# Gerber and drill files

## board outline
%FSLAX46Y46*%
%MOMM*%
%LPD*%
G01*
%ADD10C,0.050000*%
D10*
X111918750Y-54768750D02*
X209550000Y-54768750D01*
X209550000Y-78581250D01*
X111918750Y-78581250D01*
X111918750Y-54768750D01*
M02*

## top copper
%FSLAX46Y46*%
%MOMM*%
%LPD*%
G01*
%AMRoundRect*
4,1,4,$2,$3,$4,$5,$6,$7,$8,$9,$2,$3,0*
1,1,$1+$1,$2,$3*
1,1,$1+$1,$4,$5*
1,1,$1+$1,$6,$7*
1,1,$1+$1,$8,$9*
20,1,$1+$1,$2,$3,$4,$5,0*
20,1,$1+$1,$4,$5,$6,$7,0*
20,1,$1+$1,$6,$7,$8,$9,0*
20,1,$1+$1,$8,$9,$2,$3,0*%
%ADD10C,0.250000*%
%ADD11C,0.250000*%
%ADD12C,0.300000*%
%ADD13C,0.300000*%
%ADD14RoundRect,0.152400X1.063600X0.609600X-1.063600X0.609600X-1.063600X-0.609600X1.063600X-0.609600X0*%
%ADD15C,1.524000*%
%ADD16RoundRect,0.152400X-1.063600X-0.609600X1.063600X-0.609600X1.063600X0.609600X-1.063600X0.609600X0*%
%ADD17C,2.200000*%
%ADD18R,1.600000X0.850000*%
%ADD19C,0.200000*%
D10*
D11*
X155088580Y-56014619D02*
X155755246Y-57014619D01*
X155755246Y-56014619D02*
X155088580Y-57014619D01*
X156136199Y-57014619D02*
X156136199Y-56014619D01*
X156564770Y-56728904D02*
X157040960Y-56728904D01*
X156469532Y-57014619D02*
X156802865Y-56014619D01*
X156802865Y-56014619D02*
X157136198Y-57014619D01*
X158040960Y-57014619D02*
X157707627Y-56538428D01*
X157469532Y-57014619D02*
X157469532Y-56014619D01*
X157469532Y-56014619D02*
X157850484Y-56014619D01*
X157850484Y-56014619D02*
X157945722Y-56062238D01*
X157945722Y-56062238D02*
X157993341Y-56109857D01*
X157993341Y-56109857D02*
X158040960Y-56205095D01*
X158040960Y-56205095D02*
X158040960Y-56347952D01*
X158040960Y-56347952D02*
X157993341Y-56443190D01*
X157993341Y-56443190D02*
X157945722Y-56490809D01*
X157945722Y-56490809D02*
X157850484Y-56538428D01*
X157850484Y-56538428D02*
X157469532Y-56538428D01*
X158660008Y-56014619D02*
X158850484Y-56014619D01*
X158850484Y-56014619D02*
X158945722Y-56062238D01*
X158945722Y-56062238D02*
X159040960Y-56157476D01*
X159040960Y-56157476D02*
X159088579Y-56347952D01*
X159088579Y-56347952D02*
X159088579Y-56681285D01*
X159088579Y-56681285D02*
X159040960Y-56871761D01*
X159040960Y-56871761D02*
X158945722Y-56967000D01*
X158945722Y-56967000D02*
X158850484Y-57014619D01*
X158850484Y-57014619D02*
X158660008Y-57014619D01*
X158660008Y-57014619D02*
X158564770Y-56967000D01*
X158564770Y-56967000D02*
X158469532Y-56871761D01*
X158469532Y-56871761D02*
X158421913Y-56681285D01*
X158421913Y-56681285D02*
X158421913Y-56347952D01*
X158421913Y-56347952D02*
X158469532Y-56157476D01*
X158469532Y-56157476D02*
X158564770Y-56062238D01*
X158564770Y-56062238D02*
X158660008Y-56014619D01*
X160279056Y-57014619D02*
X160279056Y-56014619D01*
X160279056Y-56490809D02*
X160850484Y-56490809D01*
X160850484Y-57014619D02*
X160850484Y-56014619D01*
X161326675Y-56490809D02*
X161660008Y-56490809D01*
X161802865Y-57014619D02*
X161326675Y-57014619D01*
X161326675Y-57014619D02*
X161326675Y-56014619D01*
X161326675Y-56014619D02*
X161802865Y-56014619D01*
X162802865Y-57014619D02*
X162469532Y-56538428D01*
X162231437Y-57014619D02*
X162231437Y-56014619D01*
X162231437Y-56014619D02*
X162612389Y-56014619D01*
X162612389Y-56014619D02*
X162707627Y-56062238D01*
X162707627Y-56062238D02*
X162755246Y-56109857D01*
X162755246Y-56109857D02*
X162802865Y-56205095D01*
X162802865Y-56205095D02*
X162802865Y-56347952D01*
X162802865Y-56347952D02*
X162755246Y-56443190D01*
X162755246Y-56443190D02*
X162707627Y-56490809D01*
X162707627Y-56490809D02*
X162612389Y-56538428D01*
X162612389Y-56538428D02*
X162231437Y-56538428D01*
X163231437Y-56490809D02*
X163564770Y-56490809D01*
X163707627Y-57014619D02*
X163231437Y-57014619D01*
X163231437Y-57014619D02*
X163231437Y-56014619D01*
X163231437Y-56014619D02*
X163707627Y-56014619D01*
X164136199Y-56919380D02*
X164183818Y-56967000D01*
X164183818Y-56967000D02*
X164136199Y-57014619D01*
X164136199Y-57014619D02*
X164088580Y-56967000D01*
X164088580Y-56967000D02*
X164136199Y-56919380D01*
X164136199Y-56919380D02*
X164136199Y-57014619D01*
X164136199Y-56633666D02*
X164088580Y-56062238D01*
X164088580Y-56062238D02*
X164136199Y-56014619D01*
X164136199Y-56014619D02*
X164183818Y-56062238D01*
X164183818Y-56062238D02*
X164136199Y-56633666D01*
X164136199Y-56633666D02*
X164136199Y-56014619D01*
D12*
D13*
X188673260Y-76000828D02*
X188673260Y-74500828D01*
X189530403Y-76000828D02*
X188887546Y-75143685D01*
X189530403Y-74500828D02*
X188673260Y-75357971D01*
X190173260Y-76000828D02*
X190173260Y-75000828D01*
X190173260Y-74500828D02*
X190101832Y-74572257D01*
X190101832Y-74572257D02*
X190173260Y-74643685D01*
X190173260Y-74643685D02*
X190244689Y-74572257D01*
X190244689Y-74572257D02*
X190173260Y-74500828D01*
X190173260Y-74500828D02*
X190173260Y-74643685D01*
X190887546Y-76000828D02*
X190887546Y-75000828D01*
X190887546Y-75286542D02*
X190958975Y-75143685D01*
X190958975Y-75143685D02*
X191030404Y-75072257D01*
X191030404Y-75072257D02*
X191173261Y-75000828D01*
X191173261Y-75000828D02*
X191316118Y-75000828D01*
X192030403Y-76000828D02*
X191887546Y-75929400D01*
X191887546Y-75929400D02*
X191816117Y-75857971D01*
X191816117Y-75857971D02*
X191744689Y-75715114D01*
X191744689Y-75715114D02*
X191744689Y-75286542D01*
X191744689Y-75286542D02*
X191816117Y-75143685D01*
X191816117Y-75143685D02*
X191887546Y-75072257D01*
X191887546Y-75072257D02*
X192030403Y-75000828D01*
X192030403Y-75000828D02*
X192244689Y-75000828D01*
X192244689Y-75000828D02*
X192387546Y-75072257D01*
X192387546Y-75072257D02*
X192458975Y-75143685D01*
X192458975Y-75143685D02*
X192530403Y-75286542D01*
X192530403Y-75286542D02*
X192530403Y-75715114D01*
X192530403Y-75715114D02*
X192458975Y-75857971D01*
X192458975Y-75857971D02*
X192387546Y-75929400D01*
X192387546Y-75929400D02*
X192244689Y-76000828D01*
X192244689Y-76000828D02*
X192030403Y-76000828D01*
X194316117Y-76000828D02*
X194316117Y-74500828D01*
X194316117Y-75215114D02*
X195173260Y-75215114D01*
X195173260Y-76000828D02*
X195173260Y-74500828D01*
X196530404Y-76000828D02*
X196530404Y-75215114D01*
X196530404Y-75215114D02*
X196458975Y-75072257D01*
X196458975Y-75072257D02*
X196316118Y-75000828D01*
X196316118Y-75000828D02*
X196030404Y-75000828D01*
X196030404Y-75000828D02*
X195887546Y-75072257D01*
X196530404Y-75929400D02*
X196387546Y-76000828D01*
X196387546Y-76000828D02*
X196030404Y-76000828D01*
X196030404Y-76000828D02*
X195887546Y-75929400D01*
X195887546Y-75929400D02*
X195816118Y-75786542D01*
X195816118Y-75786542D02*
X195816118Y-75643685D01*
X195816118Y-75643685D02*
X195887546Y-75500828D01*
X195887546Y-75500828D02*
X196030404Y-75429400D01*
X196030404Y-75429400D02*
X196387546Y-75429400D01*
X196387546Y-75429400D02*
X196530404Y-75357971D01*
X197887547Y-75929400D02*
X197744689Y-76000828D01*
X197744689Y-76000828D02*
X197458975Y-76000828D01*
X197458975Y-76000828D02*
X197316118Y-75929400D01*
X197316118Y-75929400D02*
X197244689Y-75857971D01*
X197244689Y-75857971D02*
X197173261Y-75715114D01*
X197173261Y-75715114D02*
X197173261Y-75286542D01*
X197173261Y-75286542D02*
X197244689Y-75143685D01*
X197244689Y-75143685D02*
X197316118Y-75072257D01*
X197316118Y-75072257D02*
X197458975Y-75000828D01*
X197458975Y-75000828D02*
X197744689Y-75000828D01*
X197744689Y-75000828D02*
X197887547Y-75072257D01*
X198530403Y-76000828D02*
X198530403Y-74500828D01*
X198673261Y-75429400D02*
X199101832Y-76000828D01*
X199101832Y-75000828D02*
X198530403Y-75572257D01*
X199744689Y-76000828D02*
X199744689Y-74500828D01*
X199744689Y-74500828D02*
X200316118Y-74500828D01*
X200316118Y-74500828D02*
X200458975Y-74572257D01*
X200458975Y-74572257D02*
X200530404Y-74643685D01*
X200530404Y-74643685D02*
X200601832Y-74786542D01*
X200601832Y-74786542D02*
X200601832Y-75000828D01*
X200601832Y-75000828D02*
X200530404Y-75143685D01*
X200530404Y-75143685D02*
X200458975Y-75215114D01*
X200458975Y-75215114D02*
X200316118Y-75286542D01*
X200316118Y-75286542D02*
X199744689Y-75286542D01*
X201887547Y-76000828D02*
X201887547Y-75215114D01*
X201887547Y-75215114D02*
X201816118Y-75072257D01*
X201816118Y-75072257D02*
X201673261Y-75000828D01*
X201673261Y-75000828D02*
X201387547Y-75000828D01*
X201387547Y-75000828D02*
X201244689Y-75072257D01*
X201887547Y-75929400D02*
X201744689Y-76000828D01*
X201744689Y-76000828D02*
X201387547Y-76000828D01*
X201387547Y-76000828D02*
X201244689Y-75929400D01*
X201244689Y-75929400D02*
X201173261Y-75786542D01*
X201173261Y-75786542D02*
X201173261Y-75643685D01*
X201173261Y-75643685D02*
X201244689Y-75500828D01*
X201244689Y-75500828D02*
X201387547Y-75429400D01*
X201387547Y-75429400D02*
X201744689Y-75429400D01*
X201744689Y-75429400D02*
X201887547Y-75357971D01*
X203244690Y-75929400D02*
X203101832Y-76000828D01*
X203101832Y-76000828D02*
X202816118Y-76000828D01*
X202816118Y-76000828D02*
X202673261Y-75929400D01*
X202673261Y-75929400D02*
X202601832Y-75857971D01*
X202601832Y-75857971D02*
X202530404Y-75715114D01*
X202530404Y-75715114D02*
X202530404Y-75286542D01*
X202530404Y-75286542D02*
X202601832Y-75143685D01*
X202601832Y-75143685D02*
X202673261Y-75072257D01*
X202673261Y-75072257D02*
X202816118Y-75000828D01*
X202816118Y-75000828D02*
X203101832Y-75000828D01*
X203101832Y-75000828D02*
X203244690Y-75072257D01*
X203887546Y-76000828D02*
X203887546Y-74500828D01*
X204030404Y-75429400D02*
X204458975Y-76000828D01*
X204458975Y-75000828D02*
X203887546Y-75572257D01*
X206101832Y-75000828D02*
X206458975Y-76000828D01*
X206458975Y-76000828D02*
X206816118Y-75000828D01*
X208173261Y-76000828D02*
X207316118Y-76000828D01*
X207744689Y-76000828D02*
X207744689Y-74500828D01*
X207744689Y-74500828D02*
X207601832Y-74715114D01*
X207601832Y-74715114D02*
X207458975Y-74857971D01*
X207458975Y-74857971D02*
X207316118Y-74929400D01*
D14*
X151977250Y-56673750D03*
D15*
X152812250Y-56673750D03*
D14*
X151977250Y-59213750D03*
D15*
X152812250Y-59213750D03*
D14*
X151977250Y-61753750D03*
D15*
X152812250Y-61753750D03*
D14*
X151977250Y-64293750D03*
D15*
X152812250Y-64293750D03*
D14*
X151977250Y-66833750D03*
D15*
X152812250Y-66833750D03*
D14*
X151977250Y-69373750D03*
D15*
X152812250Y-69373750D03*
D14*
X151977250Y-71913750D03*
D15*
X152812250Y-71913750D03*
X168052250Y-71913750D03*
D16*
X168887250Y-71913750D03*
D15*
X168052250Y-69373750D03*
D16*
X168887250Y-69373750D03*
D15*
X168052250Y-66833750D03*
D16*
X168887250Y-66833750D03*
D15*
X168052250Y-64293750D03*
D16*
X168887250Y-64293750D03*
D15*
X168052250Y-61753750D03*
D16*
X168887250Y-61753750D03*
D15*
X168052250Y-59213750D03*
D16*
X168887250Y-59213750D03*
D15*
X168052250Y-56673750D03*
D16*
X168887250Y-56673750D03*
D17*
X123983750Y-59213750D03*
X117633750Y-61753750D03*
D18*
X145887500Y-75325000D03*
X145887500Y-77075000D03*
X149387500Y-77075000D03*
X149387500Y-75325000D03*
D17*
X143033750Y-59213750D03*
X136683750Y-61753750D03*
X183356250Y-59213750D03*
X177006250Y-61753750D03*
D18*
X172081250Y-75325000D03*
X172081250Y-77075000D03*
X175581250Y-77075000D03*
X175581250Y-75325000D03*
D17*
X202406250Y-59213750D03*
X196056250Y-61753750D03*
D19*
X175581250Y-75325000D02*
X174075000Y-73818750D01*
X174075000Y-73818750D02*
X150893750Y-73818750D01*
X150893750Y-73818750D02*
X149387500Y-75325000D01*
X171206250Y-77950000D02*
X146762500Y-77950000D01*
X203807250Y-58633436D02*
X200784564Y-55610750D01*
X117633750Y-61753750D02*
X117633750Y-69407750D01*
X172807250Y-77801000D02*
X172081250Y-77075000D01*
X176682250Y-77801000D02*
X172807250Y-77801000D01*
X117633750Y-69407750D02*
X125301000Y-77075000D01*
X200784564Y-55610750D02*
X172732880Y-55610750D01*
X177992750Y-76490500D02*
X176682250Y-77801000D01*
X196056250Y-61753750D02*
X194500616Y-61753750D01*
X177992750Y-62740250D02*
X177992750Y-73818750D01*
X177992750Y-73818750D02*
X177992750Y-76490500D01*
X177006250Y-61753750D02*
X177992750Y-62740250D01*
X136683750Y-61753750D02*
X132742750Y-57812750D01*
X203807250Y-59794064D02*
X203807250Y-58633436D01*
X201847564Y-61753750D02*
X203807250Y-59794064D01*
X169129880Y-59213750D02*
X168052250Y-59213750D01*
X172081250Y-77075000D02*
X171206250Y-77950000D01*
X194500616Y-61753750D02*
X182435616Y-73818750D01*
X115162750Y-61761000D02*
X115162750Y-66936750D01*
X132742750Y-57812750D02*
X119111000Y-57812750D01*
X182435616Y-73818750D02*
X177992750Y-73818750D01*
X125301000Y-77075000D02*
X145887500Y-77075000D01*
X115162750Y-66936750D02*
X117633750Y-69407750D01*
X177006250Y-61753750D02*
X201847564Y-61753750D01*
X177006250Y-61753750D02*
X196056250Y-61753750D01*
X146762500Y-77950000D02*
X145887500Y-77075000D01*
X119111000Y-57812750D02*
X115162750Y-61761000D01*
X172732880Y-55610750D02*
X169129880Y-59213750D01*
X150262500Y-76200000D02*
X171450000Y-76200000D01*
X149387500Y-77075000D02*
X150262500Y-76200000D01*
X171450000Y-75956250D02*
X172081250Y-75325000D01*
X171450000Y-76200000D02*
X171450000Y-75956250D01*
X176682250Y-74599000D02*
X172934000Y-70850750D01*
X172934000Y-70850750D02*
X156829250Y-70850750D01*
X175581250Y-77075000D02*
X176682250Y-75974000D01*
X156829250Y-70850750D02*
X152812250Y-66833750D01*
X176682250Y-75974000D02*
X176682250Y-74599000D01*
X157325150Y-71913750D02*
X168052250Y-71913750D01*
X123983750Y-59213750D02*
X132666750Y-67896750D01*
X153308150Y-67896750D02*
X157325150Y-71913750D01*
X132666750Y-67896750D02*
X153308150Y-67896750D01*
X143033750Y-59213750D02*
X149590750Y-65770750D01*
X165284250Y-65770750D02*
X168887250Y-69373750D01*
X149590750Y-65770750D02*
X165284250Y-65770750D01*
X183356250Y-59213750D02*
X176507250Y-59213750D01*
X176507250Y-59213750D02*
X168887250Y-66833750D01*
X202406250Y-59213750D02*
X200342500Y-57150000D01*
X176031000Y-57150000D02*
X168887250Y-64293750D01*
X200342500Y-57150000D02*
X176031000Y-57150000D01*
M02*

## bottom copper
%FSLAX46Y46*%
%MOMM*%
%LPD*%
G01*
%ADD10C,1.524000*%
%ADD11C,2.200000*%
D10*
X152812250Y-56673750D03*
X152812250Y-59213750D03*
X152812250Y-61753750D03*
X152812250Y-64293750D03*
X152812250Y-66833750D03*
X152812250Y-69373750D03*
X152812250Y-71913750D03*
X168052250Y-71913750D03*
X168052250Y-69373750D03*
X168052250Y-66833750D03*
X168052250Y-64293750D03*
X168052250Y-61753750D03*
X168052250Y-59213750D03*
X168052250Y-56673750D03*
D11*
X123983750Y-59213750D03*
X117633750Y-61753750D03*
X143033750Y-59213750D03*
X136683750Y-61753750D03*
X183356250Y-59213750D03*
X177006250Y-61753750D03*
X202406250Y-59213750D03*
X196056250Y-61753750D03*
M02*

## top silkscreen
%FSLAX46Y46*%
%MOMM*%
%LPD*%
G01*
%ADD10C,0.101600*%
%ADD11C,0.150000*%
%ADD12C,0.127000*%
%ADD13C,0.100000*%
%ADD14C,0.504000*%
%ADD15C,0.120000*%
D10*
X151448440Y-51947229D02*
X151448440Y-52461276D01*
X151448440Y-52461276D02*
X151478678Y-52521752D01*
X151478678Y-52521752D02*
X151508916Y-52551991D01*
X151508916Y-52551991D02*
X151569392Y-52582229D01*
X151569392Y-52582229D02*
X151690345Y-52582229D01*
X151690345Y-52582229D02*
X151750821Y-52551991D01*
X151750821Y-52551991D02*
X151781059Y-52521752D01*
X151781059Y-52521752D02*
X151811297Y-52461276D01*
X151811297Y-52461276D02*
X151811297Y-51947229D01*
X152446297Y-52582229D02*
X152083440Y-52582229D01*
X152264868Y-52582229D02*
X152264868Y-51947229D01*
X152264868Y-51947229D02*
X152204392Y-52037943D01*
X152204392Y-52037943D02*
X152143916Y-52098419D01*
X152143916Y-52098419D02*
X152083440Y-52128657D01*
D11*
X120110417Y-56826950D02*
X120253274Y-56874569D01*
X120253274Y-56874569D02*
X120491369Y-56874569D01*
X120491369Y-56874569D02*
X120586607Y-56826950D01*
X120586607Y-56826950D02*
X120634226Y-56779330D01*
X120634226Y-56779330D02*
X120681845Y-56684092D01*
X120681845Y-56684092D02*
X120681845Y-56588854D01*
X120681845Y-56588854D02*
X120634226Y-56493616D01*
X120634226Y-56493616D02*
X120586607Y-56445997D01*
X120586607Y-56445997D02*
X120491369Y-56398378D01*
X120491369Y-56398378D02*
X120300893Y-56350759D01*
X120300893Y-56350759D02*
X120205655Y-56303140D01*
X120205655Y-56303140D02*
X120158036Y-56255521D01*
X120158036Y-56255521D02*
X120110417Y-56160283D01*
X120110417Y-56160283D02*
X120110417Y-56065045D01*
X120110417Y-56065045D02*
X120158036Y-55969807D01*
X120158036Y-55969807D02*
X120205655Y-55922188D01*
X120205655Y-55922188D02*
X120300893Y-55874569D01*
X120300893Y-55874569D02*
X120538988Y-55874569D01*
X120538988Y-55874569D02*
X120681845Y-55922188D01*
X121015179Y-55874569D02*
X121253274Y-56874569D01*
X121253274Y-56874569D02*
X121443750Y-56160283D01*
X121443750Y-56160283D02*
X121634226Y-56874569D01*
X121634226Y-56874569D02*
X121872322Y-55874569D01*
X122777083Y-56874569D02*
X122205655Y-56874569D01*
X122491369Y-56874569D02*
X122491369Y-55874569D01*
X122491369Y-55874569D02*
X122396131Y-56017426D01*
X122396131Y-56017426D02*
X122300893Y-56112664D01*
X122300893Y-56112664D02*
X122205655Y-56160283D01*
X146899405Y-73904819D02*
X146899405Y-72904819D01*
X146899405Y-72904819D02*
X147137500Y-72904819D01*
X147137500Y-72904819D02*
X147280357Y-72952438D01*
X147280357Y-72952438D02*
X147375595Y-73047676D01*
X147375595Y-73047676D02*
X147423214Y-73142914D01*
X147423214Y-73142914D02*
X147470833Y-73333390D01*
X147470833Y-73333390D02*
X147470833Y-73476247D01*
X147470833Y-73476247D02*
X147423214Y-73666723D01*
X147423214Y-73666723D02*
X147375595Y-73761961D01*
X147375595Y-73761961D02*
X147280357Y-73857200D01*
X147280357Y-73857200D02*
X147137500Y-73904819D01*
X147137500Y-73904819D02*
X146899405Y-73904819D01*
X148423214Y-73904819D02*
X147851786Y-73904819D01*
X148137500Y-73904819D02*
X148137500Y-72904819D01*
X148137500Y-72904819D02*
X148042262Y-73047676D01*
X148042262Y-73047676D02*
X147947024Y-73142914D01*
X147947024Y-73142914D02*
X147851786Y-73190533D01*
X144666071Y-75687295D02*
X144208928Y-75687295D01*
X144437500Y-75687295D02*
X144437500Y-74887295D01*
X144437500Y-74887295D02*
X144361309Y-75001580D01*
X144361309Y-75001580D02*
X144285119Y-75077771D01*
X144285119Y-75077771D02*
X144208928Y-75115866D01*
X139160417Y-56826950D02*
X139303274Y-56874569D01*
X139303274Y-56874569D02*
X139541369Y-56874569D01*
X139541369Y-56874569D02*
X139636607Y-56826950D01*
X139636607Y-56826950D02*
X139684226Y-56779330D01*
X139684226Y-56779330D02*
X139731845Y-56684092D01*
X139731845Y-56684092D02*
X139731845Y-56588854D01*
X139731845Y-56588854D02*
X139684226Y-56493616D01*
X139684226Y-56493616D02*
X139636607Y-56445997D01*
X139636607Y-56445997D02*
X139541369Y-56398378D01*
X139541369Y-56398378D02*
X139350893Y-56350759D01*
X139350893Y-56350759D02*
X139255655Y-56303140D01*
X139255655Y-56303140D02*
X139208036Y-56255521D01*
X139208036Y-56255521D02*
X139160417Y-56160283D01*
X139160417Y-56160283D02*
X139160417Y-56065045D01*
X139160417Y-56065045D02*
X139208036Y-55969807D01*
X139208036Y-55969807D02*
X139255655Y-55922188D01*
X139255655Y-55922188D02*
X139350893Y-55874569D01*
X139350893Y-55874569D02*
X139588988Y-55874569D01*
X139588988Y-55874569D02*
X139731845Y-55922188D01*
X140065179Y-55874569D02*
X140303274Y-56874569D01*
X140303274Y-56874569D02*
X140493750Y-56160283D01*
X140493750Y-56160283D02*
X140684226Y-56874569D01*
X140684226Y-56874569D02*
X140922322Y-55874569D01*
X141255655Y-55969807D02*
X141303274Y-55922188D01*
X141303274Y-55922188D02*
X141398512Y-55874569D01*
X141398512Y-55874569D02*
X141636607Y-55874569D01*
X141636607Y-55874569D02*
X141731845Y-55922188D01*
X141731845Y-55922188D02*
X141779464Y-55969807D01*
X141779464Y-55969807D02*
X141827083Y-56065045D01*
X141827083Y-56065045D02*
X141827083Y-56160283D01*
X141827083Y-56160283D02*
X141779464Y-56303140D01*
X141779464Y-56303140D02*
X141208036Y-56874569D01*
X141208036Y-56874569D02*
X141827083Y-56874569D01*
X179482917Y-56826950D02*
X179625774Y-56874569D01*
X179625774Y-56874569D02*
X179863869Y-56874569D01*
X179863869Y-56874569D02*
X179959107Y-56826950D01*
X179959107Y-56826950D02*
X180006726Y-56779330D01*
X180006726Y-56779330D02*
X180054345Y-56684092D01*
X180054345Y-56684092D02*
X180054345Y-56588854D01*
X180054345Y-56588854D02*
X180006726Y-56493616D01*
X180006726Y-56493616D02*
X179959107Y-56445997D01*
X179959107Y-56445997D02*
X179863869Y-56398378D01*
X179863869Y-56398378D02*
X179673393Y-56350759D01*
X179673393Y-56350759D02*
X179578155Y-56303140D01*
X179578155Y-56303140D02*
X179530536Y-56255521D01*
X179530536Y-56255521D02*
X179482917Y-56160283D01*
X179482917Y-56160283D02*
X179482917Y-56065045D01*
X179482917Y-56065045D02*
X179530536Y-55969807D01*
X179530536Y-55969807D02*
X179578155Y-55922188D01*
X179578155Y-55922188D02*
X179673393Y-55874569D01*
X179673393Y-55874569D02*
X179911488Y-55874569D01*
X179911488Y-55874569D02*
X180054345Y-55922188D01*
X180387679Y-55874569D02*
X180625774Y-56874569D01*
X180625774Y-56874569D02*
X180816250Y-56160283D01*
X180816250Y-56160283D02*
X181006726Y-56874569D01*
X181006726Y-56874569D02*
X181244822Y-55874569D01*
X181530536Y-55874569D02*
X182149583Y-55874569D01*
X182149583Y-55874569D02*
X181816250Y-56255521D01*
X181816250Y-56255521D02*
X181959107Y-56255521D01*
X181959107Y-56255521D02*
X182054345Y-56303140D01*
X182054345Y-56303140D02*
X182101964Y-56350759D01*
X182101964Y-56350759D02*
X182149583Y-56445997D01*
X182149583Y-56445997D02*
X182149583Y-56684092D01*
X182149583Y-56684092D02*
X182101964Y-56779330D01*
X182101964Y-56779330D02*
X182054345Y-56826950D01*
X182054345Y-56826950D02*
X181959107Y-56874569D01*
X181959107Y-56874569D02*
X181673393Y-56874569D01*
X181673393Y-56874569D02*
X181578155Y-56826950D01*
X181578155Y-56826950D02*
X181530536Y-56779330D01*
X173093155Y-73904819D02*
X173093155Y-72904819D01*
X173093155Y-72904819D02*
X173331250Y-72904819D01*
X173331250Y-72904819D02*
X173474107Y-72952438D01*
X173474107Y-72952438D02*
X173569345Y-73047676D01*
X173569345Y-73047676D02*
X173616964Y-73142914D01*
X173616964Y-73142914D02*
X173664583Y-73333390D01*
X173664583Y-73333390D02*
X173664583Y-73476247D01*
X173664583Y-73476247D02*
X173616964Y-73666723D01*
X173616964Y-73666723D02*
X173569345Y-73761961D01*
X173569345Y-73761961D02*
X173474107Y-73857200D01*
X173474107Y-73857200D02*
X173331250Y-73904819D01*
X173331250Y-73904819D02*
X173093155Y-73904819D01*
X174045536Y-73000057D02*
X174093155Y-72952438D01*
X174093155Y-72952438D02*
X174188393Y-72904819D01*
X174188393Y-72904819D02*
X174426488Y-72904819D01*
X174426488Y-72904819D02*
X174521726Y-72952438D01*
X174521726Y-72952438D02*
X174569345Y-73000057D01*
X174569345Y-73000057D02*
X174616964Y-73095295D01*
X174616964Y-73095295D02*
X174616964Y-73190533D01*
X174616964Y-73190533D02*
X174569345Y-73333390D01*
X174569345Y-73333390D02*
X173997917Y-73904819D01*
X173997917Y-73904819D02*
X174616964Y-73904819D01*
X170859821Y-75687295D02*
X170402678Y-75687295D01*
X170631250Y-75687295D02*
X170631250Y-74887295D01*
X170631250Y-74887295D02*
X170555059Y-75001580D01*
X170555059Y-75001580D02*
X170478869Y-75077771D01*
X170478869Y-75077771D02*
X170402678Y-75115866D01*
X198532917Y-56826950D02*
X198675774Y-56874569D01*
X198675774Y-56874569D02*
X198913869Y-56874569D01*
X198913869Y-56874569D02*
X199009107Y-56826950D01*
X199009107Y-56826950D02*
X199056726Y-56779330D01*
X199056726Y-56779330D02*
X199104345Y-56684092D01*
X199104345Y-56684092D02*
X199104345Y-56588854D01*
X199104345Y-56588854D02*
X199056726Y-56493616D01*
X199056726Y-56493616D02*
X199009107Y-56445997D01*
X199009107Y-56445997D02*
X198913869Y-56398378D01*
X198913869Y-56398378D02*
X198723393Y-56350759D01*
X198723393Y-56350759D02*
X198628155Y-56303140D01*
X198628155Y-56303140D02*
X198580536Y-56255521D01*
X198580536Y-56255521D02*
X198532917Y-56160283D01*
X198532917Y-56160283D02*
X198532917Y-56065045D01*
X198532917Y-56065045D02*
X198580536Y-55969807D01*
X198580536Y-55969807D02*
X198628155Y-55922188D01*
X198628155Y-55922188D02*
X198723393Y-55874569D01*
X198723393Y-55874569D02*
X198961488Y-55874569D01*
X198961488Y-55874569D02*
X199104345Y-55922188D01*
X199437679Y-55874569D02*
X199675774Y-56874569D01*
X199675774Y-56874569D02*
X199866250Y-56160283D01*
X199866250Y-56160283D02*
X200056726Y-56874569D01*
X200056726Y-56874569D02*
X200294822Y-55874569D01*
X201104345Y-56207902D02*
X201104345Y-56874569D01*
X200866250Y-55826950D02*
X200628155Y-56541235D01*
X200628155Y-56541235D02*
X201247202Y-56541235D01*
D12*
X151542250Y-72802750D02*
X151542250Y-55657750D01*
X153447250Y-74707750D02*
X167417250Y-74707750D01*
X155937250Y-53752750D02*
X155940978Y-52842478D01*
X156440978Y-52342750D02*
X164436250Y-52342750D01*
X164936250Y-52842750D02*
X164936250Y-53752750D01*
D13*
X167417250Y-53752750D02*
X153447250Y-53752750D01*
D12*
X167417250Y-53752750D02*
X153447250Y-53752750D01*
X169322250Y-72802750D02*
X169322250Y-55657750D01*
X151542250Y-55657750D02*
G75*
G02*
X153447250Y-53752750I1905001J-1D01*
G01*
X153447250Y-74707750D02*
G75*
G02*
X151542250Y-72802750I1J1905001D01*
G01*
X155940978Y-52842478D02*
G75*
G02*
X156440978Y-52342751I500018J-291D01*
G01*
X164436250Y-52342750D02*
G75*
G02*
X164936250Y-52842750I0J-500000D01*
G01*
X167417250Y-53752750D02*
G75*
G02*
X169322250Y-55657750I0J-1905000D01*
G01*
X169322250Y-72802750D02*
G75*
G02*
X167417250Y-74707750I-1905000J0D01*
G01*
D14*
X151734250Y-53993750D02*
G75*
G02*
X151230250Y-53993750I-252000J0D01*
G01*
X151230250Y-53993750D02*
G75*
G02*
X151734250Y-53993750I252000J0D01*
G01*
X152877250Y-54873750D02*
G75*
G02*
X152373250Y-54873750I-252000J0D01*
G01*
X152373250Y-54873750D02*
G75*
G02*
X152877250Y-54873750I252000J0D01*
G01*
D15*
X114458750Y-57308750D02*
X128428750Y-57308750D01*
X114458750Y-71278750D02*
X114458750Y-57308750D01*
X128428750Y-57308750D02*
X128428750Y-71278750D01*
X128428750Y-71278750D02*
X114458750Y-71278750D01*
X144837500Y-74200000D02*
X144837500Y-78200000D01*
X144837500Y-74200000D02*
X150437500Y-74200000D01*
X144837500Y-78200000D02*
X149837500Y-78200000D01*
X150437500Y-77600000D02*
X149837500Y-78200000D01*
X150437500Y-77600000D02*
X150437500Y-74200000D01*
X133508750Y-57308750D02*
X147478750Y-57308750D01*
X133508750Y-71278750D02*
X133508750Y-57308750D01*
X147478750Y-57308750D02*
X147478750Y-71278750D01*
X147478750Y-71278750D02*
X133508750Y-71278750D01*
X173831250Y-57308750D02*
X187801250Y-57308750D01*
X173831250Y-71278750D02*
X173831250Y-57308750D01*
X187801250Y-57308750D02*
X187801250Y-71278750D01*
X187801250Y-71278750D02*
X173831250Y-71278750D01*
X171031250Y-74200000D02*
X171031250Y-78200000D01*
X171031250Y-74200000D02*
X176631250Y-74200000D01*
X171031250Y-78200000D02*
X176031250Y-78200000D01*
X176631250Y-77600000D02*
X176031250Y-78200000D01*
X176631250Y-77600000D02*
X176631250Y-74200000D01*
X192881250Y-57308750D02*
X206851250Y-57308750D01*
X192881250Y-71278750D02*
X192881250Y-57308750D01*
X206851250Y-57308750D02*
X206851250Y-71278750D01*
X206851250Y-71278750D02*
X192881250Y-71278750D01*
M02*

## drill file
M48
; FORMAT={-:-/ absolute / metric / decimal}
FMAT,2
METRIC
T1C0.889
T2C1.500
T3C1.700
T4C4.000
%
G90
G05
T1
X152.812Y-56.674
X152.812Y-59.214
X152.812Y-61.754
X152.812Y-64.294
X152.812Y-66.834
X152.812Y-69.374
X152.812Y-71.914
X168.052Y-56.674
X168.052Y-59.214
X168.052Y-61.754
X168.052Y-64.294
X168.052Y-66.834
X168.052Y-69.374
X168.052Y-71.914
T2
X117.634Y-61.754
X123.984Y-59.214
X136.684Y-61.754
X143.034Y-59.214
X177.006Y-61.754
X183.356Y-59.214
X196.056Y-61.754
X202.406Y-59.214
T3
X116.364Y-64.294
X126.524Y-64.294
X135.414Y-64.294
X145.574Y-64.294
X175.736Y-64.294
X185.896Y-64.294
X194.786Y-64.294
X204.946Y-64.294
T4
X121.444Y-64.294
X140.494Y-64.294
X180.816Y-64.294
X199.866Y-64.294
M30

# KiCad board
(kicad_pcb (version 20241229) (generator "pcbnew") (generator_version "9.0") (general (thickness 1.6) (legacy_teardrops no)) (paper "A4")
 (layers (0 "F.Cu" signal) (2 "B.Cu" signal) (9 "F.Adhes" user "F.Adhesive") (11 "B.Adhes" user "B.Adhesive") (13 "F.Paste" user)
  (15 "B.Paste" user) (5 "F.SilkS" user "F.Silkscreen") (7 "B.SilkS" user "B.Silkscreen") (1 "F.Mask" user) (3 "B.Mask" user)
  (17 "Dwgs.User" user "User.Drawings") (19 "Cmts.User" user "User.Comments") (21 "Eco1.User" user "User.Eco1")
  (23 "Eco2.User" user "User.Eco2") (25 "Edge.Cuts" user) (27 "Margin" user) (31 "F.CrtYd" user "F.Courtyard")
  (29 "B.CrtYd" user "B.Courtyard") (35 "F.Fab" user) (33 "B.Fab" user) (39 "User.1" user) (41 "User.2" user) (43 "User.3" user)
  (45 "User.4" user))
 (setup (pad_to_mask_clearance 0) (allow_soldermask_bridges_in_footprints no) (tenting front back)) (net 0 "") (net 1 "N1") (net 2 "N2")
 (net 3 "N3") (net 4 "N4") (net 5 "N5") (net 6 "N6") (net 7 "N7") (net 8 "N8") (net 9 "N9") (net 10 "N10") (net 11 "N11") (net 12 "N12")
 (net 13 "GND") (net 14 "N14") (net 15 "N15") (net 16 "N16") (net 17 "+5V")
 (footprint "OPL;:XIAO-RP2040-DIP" (layer "F.Cu") (at 160.43225 64.29375)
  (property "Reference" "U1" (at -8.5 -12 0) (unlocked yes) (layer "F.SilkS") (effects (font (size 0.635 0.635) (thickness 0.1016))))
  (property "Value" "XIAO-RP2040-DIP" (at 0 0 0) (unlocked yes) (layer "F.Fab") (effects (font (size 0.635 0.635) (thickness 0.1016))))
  (fp_line (start -8.89 8.509) (end -8.89 -8.636) (stroke (width 0.127) (type solid)) (layer "F.SilkS"))
  (fp_line (start -6.985 10.414) (end 6.985 10.414) (stroke (width 0.127) (type solid)) (layer "F.SilkS"))
  (fp_line (start -4.495 -10.541) (end -4.491272 -11.451272) (stroke (width 0.127) (type solid)) (layer "F.SilkS"))
  (fp_line (start -3.991272 -11.951) (end 4.004 -11.951) (stroke (width 0.127) (type solid)) (layer "F.SilkS"))
  (fp_line (start 4.504 -11.451) (end 4.504 -10.541) (stroke (width 0.127) (type solid)) (layer "F.SilkS"))
  (fp_line (start 6.985 -10.541) (end -6.985 -10.541) (stroke (width 0.1) (type solid)) (layer "F.SilkS"))
  (fp_line (start 6.985 -10.541) (end -6.985 -10.541) (stroke (width 0.127) (type solid)) (layer "F.SilkS"))
  (fp_line (start 8.89 8.509) (end 8.89 -8.636) (stroke (width 0.127) (type solid)) (layer "F.SilkS"))
  (fp_arc (start -8.89 -8.636) (mid -8.332038 -9.983038) (end -6.985 -10.541) (stroke (width 0.127) (type solid)) (layer "F.SilkS"))
  (fp_arc (start -6.985 10.414) (mid -8.332038 9.856038) (end -8.89 8.509) (stroke (width 0.127) (type solid)) (layer "F.SilkS"))
  (fp_arc (start -4.491272 -11.451272) (mid -4.344728 -11.80464) (end -3.991272 -11.951) (stroke (width 0.127) (type default))
   (layer "F.SilkS"))
  (fp_arc (start 4.004 -11.951) (mid 4.357553 -11.804553) (end 4.504 -11.451) (stroke (width 0.127) (type default)) (layer "F.SilkS"))
  (fp_arc (start 6.985 -10.541) (mid 8.332038 -9.983038) (end 8.89 -8.636) (stroke (width 0.127) (type solid)) (layer "F.SilkS"))
  (fp_arc (start 8.89 8.509) (mid 8.332038 9.856038) (end 6.985 10.414) (stroke (width 0.127) (type solid)) (layer "F.SilkS"))
  (fp_circle (center -8.95 -10.3) (end -8.95 -10.554) (stroke (width 0.5) (type solid)) (fill yes) (layer "F.SilkS"))
  (fp_circle (center -7.807 -9.42) (end -7.807 -9.674) (stroke (width 0.5) (type solid)) (fill yes) (layer "F.SilkS"))
  (pad "1" smd roundrect (at -8.455 -7.62 180) (size 2.432 1.524) (layers "F.Cu" "F.Mask") (roundrect_rratio 0.1) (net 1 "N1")
   (thermal_bridge_angle 45))
  (pad "1" thru_hole circle (at -7.62 -7.62 180) (size 1.524 1.524) (drill 0.889) (layers "*.Cu" "*.Mask") (remove_unused_layers no)
   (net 1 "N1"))
  (pad "2" smd roundrect (at -8.455 -5.08 180) (size 2.432 1.524) (layers "F.Cu" "F.Mask") (roundrect_rratio 0.1) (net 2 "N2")
   (thermal_bridge_angle 45))
  (pad "2" thru_hole circle (at -7.62 -5.08 180) (size 1.524 1.524) (drill 0.889) (layers "*.Cu" "*.Mask") (remove_unused_layers no)
   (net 2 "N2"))
  (pad "3" smd roundrect (at -8.455 -2.54 180) (size 2.432 1.524) (layers "F.Cu" "F.Mask") (roundrect_rratio 0.1) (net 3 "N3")
   (thermal_bridge_angle 45))
  (pad "3" thru_hole circle (at -7.62 -2.54 180) (size 1.524 1.524) (drill 0.889) (layers "*.Cu" "*.Mask") (remove_unused_layers no)
   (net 3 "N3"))
  (pad "4" smd roundrect (at -8.455 0 180) (size 2.432 1.524) (layers "F.Cu" "F.Mask") (roundrect_rratio 0.1) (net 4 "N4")
   (thermal_bridge_angle 45))
  (pad "4" thru_hole circle (at -7.62 0 180) (size 1.524 1.524) (drill 0.889) (layers "*.Cu" "*.Mask") (remove_unused_layers no)
   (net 4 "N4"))
  (pad "5" smd roundrect (at -8.455 2.54 180) (size 2.432 1.524) (layers "F.Cu" "F.Mask") (roundrect_rratio 0.1) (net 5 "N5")
   (thermal_bridge_angle 45))
  (pad "5" thru_hole circle (at -7.62 2.54 180) (size 1.524 1.524) (drill 0.889) (layers "*.Cu" "*.Mask") (remove_unused_layers no)
   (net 5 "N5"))
  (pad "6" smd roundrect (at -8.455 5.08 180) (size 2.432 1.524) (layers "F.Cu" "F.Mask") (roundrect_rratio 0.1) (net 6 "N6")
   (thermal_bridge_angle 45))
  (pad "6" thru_hole circle (at -7.62 5.08 180) (size 1.524 1.524) (drill 0.889) (layers "*.Cu" "*.Mask") (remove_unused_layers no)
   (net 6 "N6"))
  (pad "7" smd roundrect (at -8.455 7.62 180) (size 2.432 1.524) (layers "F.Cu" "F.Mask") (roundrect_rratio 0.1) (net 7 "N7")
   (thermal_bridge_angle 45))
  (pad "7" thru_hole circle (at -7.62 7.62 180) (size 1.524 1.524) (drill 0.889) (layers "*.Cu" "*.Mask") (remove_unused_layers no)
   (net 7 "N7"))
  (pad "8" thru_hole circle (at 7.62 7.62) (size 1.524 1.524) (drill 0.889) (layers "*.Cu" "*.Mask") (remove_unused_layers no) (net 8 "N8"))
  (pad "8" smd roundrect (at 8.455 7.62) (size 2.432 1.524) (layers "F.Cu" "F.Mask") (roundrect_rratio 0.1) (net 8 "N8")
   (thermal_bridge_angle 45))
  (pad "9" thru_hole circle (at 7.62 5.08) (size 1.524 1.524) (drill 0.889) (layers "*.Cu" "*.Mask") (remove_unused_layers no) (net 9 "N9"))
  (pad "9" smd roundrect (at 8.455 5.08) (size 2.432 1.524) (layers "F.Cu" "F.Mask") (roundrect_rratio 0.1) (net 9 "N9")
   (thermal_bridge_angle 45))
  (pad "10" thru_hole circle (at 7.62 2.54) (size 1.524 1.524) (drill 0.889) (layers "*.Cu" "*.Mask") (remove_unused_layers no)
   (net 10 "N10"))
  (pad "10" smd roundrect (at 8.455 2.54) (size 2.432 1.524) (layers "F.Cu" "F.Mask") (roundrect_rratio 0.1) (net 10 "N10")
   (thermal_bridge_angle 45))
  (pad "11" thru_hole circle (at 7.62 0) (size 1.524 1.524) (drill 0.889) (layers "*.Cu" "*.Mask") (remove_unused_layers no) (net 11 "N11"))
  (pad "11" smd roundrect (at 8.455 0) (size 2.432 1.524) (layers "F.Cu" "F.Mask") (roundrect_rratio 0.1) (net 11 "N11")
   (thermal_bridge_angle 45))
  (pad "12" thru_hole circle (at 7.62 -2.54) (size 1.524 1.524) (drill 0.889) (layers "*.Cu" "*.Mask") (remove_unused_layers no)
   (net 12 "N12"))
  (pad "12" smd roundrect (at 8.455 -2.54) (size 2.432 1.524) (layers "F.Cu" "F.Mask") (roundrect_rratio 0.1) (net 12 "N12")
   (thermal_bridge_angle 45))
  (pad "13" thru_hole circle (at 7.62 -5.08) (size 1.524 1.524) (drill 0.889) (layers "*.Cu" "*.Mask") (remove_unused_layers no)
   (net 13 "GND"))
  (pad "13" smd roundrect (at 8.455 -5.08) (size 2.432 1.524) (layers "F.Cu" "F.Mask") (roundrect_rratio 0.1) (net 13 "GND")
   (thermal_bridge_angle 45))
  (pad "14" thru_hole circle (at 7.62 -7.62) (size 1.524 1.524) (drill 0.889) (layers "*.Cu" "*.Mask") (remove_unused_layers no)
   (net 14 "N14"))
  (pad "14" smd roundrect (at 8.455 -7.62) (size 2.432 1.524) (layers "F.Cu" "F.Mask") (roundrect_rratio 0.1) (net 14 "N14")
   (thermal_bridge_angle 45)))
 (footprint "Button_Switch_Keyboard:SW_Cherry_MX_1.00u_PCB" (layer "F.Cu") (at 123.98375 59.21375)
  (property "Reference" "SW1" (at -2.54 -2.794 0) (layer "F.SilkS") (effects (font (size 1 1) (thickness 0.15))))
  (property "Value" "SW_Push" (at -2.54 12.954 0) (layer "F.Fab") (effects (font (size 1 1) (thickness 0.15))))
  (fp_line (start -9.525 -1.905) (end 4.445 -1.905) (stroke (width 0.12) (type solid)) (layer "F.SilkS"))
  (fp_line (start -9.525 12.065) (end -9.525 -1.905) (stroke (width 0.12) (type solid)) (layer "F.SilkS"))
  (fp_line (start 4.445 -1.905) (end 4.445 12.065) (stroke (width 0.12) (type solid)) (layer "F.SilkS"))
  (fp_line (start 4.445 12.065) (end -9.525 12.065) (stroke (width 0.12) (type solid)) (layer "F.SilkS"))
  (pad "" np_thru_hole circle (at -7.62 5.08) (size 1.7 1.7) (drill 1.7) (layers "*.Cu" "*.Mask"))
  (pad "" np_thru_hole circle (at -2.54 5.08) (size 4 4) (drill 4) (layers "*.Cu" "*.Mask"))
  (pad "" np_thru_hole circle (at 2.54 5.08) (size 1.7 1.7) (drill 1.7) (layers "*.Cu" "*.Mask"))
  (pad "1" thru_hole circle (at 0 0) (size 2.2 2.2) (drill 1.5) (layers "*.Cu" "*.Mask") (remove_unused_layers no) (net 8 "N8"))
  (pad "2" thru_hole circle (at -6.35 2.54) (size 2.2 2.2) (drill 1.5) (layers "*.Cu" "*.Mask") (remove_unused_layers no) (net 13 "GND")))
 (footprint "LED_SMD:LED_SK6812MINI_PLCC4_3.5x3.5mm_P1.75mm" (layer "F.Cu") (at 147.6375 76.2)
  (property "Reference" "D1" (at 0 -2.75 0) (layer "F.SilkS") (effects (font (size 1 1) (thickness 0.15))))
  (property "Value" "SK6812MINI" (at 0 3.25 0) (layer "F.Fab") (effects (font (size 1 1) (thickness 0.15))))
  (fp_line (start -2.8 -2) (end -2.8 2) (stroke (width 0.12) (type default)) (layer "F.SilkS"))
  (fp_line (start -2.8 -2) (end 2.8 -2) (stroke (width 0.12) (type solid)) (layer "F.SilkS"))
  (fp_line (start -2.8 2) (end 2.2 2) (stroke (width 0.12) (type solid)) (layer "F.SilkS"))
  (fp_line (start 2.8 1.4) (end 2.2 2) (stroke (width 0.12) (type default)) (layer "F.SilkS"))
  (fp_line (start 2.8 1.4) (end 2.8 -2) (stroke (width 0.12) (type solid)) (layer "F.SilkS"))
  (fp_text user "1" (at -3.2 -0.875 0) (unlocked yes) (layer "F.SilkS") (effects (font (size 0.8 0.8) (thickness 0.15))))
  (pad "1" smd rect (at -1.75 -0.875) (size 1.6 0.85) (layers "F.Cu" "F.Mask" "F.Paste") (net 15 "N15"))
  (pad "2" smd rect (at -1.75 0.875) (size 1.6 0.85) (layers "F.Cu" "F.Mask" "F.Paste") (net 13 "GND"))
  (pad "3" smd rect (at 1.75 0.875) (size 1.6 0.85) (layers "F.Cu" "F.Mask" "F.Paste") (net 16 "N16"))
  (pad "4" smd rect (at 1.75 -0.875) (size 1.6 0.85) (layers "F.Cu" "F.Mask" "F.Paste") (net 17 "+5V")))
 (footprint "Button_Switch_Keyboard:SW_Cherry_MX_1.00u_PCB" (layer "F.Cu") (at 143.03375 59.21375)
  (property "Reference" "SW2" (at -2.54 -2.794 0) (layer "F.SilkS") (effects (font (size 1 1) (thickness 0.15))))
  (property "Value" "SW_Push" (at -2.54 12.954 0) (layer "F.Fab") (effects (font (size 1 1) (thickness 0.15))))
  (fp_line (start -9.525 -1.905) (end 4.445 -1.905) (stroke (width 0.12) (type solid)) (layer "F.SilkS"))
  (fp_line (start -9.525 12.065) (end -9.525 -1.905) (stroke (width 0.12) (type solid)) (layer "F.SilkS"))
  (fp_line (start 4.445 -1.905) (end 4.445 12.065) (stroke (width 0.12) (type solid)) (layer "F.SilkS"))
  (fp_line (start 4.445 12.065) (end -9.525 12.065) (stroke (width 0.12) (type solid)) (layer "F.SilkS"))
  (pad "" np_thru_hole circle (at -7.62 5.08) (size 1.7 1.7) (drill 1.7) (layers "*.Cu" "*.Mask"))
  (pad "" np_thru_hole circle (at -2.54 5.08) (size 4 4) (drill 4) (layers "*.Cu" "*.Mask"))
  (pad "" np_thru_hole circle (at 2.54 5.08) (size 1.7 1.7) (drill 1.7) (layers "*.Cu" "*.Mask"))
  (pad "1" thru_hole circle (at 0 0) (size 2.2 2.2) (drill 1.5) (layers "*.Cu" "*.Mask") (remove_unused_layers no) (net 9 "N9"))
  (pad "2" thru_hole circle (at -6.35 2.54) (size 2.2 2.2) (drill 1.5) (layers "*.Cu" "*.Mask") (remove_unused_layers no) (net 13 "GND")))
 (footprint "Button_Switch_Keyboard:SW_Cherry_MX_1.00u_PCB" (layer "F.Cu") (at 183.35625 59.21375)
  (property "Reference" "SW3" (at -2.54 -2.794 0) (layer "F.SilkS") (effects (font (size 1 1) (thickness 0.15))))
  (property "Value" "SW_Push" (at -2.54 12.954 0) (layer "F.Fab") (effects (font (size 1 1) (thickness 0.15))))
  (fp_line (start -9.525 -1.905) (end 4.445 -1.905) (stroke (width 0.12) (type solid)) (layer "F.SilkS"))
  (fp_line (start -9.525 12.065) (end -9.525 -1.905) (stroke (width 0.12) (type solid)) (layer "F.SilkS"))
  (fp_line (start 4.445 -1.905) (end 4.445 12.065) (stroke (width 0.12) (type solid)) (layer "F.SilkS"))
  (fp_line (start 4.445 12.065) (end -9.525 12.065) (stroke (width 0.12) (type solid)) (layer "F.SilkS"))
  (pad "" np_thru_hole circle (at -7.62 5.08) (size 1.7 1.7) (drill 1.7) (layers "*.Cu" "*.Mask"))
  (pad "" np_thru_hole circle (at -2.54 5.08) (size 4 4) (drill 4) (layers "*.Cu" "*.Mask"))
  (pad "" np_thru_hole circle (at 2.54 5.08) (size 1.7 1.7) (drill 1.7) (layers "*.Cu" "*.Mask"))
  (pad "1" thru_hole circle (at 0 0) (size 2.2 2.2) (drill 1.5) (layers "*.Cu" "*.Mask") (remove_unused_layers no) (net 10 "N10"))
  (pad "2" thru_hole circle (at -6.35 2.54) (size 2.2 2.2) (drill 1.5) (layers "*.Cu" "*.Mask") (remove_unused_layers no) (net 13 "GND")))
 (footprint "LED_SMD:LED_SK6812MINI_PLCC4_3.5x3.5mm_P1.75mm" (layer "F.Cu") (at 173.83125 76.2)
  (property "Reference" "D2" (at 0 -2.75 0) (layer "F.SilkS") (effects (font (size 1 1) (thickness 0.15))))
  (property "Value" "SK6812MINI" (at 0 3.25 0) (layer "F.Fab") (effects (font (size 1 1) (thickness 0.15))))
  (fp_line (start -2.8 -2) (end -2.8 2) (stroke (width 0.12) (type default)) (layer "F.SilkS"))
  (fp_line (start -2.8 -2) (end 2.8 -2) (stroke (width 0.12) (type solid)) (layer "F.SilkS"))
  (fp_line (start -2.8 2) (end 2.2 2) (stroke (width 0.12) (type solid)) (layer "F.SilkS"))
  (fp_line (start 2.8 1.4) (end 2.2 2) (stroke (width 0.12) (type default)) (layer "F.SilkS"))
  (fp_line (start 2.8 1.4) (end 2.8 -2) (stroke (width 0.12) (type solid)) (layer "F.SilkS"))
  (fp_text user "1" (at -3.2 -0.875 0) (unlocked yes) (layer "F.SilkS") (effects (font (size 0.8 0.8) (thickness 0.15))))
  (pad "1" smd rect (at -1.75 -0.875) (size 1.6 0.85) (layers "F.Cu" "F.Mask" "F.Paste") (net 16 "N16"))
  (pad "2" smd rect (at -1.75 0.875) (size 1.6 0.85) (layers "F.Cu" "F.Mask" "F.Paste") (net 13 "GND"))
  (pad "3" smd rect (at 1.75 0.875) (size 1.6 0.85) (layers "F.Cu" "F.Mask" "F.Paste") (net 5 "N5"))
  (pad "4" smd rect (at 1.75 -0.875) (size 1.6 0.85) (layers "F.Cu" "F.Mask" "F.Paste") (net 17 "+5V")))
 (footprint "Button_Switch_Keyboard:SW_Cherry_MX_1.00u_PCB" (layer "F.Cu") (at 202.40625 59.21375)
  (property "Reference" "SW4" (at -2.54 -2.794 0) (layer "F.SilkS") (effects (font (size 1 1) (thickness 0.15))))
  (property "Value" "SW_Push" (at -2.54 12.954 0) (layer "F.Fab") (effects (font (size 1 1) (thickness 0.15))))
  (fp_line (start -9.525 -1.905) (end 4.445 -1.905) (stroke (width 0.12) (type solid)) (layer "F.SilkS"))
  (fp_line (start -9.525 12.065) (end -9.525 -1.905) (stroke (width 0.12) (type solid)) (layer "F.SilkS"))
  (fp_line (start 4.445 -1.905) (end 4.445 12.065) (stroke (width 0.12) (type solid)) (layer "F.SilkS"))
  (fp_line (start 4.445 12.065) (end -9.525 12.065) (stroke (width 0.12) (type solid)) (layer "F.SilkS"))
  (pad "" np_thru_hole circle (at -7.62 5.08) (size 1.7 1.7) (drill 1.7) (layers "*.Cu" "*.Mask"))
  (pad "" np_thru_hole circle (at -2.54 5.08) (size 4 4) (drill 4) (layers "*.Cu" "*.Mask"))
  (pad "" np_thru_hole circle (at 2.54 5.08) (size 1.7 1.7) (drill 1.7) (layers "*.Cu" "*.Mask"))
  (pad "1" thru_hole circle (at 0 0) (size 2.2 2.2) (drill 1.5) (layers "*.Cu" "*.Mask") (remove_unused_layers no) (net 11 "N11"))
  (pad "2" thru_hole circle (at -6.35 2.54) (size 2.2 2.2) (drill 1.5) (layers "*.Cu" "*.Mask") (remove_unused_layers no) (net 13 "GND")))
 (gr_rect (start 111.91875 54.76875) (end 209.55 78.58125) (stroke (width 0.05) (type default)) (fill no) (layer "Edge.Cuts"))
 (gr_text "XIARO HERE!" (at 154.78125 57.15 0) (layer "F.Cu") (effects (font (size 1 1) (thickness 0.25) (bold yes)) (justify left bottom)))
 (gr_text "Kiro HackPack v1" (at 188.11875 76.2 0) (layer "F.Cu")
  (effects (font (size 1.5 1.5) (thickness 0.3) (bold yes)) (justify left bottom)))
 (segment (start 175.58125 75.325) (end 174.075 73.81875) (width 0.2) (layer "F.Cu") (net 17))
 (segment (start 174.075 73.81875) (end 150.89375 73.81875) (width 0.2) (layer "F.Cu") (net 17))
 (segment (start 150.89375 73.81875) (end 149.3875 75.325) (width 0.2) (layer "F.Cu") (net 17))
 (segment (start 171.20625 77.95) (end 146.7625 77.95) (width 0.2) (layer "F.Cu") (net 13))
 (segment (start 203.80725 58.633436) (end 200.784564 55.61075) (width 0.2) (layer "F.Cu") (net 13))
 (segment (start 117.63375 61.75375) (end 117.63375 69.40775) (width 0.2) (layer "F.Cu") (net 13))
 (segment (start 172.80725 77.801) (end 172.08125 77.075) (width 0.2) (layer "F.Cu") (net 13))
 (segment (start 176.68225 77.801) (end 172.80725 77.801) (width 0.2) (layer "F.Cu") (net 13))
 (segment (start 117.63375 69.40775) (end 125.301 77.075) (width 0.2) (layer "F.Cu") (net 13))
 (segment (start 200.784564 55.61075) (end 172.73288 55.61075) (width 0.2) (layer "F.Cu") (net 13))
 (segment (start 177.99275 76.4905) (end 176.68225 77.801) (width 0.2) (layer "F.Cu") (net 13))
 (segment (start 196.05625 61.75375) (end 194.500616 61.75375) (width 0.2) (layer "F.Cu") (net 13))
 (segment (start 177.99275 62.74025) (end 177.99275 73.81875) (width 0.2) (layer "F.Cu") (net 13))
 (segment (start 177.99275 73.81875) (end 177.99275 76.4905) (width 0.2) (layer "F.Cu") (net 13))
 (segment (start 177.00625 61.75375) (end 177.99275 62.74025) (width 0.2) (layer "F.Cu") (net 13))
 (segment (start 136.68375 61.75375) (end 132.74275 57.81275) (width 0.2) (layer "F.Cu") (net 13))
 (segment (start 203.80725 59.794064) (end 203.80725 58.633436) (width 0.2) (layer "F.Cu") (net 13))
 (segment (start 201.847564 61.75375) (end 203.80725 59.794064) (width 0.2) (layer "F.Cu") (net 13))
 (segment (start 169.12988 59.21375) (end 168.05225 59.21375) (width 0.2) (layer "F.Cu") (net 13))
 (segment (start 172.08125 77.075) (end 171.20625 77.95) (width 0.2) (layer "F.Cu") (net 13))
 (segment (start 194.500616 61.75375) (end 182.435616 73.81875) (width 0.2) (layer "F.Cu") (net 13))
 (segment (start 115.16275 61.761) (end 115.16275 66.93675) (width 0.2) (layer "F.Cu") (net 13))
 (segment (start 132.74275 57.81275) (end 119.111 57.81275) (width 0.2) (layer "F.Cu") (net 13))
 (segment (start 182.435616 73.81875) (end 177.99275 73.81875) (width 0.2) (layer "F.Cu") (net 13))
 (segment (start 125.301 77.075) (end 145.8875 77.075) (width 0.2) (layer "F.Cu") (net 13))
 (segment (start 115.16275 66.93675) (end 117.63375 69.40775) (width 0.2) (layer "F.Cu") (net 13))
 (segment (start 177.00625 61.75375) (end 201.847564 61.75375) (width 0.2) (layer "F.Cu") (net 13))
 (segment (start 177.00625 61.75375) (end 196.05625 61.75375) (width 0.2) (layer "F.Cu") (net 13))
 (segment (start 146.7625 77.95) (end 145.8875 77.075) (width 0.2) (layer "F.Cu") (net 13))
 (segment (start 119.111 57.81275) (end 115.16275 61.761) (width 0.2) (layer "F.Cu") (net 13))
 (segment (start 172.73288 55.61075) (end 169.12988 59.21375) (width 0.2) (layer "F.Cu") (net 13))
 (segment (start 150.2625 76.2) (end 171.45 76.2) (width 0.2) (layer "F.Cu") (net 16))
 (segment (start 149.3875 77.075) (end 150.2625 76.2) (width 0.2) (layer "F.Cu") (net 16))
 (segment (start 171.45 75.95625) (end 172.08125 75.325) (width 0.2) (layer "F.Cu") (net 16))
 (segment (start 171.45 76.2) (end 171.45 75.95625) (width 0.2) (layer "F.Cu") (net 16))
 (segment (start 176.68225 74.599) (end 172.934 70.85075) (width 0.2) (layer "F.Cu") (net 5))
 (segment (start 172.934 70.85075) (end 156.82925 70.85075) (width 0.2) (layer "F.Cu") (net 5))
 (segment (start 175.58125 77.075) (end 176.68225 75.974) (width 0.2) (layer "F.Cu") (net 5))
 (segment (start 156.82925 70.85075) (end 152.81225 66.83375) (width 0.2) (layer "F.Cu") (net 5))
 (segment (start 176.68225 75.974) (end 176.68225 74.599) (width 0.2) (layer "F.Cu") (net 5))
 (segment (start 157.32515 71.91375) (end 168.05225 71.91375) (width 0.2) (layer "F.Cu") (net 8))
 (segment (start 123.98375 59.21375) (end 132.66675 67.89675) (width 0.2) (layer "F.Cu") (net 8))
 (segment (start 153.30815 67.89675) (end 157.32515 71.91375) (width 0.2) (layer "F.Cu") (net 8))
 (segment (start 132.66675 67.89675) (end 153.30815 67.89675) (width 0.2) (layer "F.Cu") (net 8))
 (segment (start 143.03375 59.21375) (end 149.59075 65.77075) (width 0.2) (layer "F.Cu") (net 9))
 (segment (start 165.28425 65.77075) (end 168.88725 69.37375) (width 0.2) (layer "F.Cu") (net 9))
 (segment (start 149.59075 65.77075) (end 165.28425 65.77075) (width 0.2) (layer "F.Cu") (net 9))
 (segment (start 183.35625 59.21375) (end 176.50725 59.21375) (width 0.2) (layer "F.Cu") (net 10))
 (segment (start 176.50725 59.21375) (end 168.88725 66.83375) (width 0.2) (layer "F.Cu") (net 10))
 (segment (start 202.40625 59.21375) (end 200.3425 57.15) (width 0.2) (layer "F.Cu") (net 11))
 (segment (start 176.031 57.15) (end 168.88725 64.29375) (width 0.2) (layer "F.Cu") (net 11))
 (segment (start 200.3425 57.15) (end 176.031 57.15) (width 0.2) (layer "F.Cu") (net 11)))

